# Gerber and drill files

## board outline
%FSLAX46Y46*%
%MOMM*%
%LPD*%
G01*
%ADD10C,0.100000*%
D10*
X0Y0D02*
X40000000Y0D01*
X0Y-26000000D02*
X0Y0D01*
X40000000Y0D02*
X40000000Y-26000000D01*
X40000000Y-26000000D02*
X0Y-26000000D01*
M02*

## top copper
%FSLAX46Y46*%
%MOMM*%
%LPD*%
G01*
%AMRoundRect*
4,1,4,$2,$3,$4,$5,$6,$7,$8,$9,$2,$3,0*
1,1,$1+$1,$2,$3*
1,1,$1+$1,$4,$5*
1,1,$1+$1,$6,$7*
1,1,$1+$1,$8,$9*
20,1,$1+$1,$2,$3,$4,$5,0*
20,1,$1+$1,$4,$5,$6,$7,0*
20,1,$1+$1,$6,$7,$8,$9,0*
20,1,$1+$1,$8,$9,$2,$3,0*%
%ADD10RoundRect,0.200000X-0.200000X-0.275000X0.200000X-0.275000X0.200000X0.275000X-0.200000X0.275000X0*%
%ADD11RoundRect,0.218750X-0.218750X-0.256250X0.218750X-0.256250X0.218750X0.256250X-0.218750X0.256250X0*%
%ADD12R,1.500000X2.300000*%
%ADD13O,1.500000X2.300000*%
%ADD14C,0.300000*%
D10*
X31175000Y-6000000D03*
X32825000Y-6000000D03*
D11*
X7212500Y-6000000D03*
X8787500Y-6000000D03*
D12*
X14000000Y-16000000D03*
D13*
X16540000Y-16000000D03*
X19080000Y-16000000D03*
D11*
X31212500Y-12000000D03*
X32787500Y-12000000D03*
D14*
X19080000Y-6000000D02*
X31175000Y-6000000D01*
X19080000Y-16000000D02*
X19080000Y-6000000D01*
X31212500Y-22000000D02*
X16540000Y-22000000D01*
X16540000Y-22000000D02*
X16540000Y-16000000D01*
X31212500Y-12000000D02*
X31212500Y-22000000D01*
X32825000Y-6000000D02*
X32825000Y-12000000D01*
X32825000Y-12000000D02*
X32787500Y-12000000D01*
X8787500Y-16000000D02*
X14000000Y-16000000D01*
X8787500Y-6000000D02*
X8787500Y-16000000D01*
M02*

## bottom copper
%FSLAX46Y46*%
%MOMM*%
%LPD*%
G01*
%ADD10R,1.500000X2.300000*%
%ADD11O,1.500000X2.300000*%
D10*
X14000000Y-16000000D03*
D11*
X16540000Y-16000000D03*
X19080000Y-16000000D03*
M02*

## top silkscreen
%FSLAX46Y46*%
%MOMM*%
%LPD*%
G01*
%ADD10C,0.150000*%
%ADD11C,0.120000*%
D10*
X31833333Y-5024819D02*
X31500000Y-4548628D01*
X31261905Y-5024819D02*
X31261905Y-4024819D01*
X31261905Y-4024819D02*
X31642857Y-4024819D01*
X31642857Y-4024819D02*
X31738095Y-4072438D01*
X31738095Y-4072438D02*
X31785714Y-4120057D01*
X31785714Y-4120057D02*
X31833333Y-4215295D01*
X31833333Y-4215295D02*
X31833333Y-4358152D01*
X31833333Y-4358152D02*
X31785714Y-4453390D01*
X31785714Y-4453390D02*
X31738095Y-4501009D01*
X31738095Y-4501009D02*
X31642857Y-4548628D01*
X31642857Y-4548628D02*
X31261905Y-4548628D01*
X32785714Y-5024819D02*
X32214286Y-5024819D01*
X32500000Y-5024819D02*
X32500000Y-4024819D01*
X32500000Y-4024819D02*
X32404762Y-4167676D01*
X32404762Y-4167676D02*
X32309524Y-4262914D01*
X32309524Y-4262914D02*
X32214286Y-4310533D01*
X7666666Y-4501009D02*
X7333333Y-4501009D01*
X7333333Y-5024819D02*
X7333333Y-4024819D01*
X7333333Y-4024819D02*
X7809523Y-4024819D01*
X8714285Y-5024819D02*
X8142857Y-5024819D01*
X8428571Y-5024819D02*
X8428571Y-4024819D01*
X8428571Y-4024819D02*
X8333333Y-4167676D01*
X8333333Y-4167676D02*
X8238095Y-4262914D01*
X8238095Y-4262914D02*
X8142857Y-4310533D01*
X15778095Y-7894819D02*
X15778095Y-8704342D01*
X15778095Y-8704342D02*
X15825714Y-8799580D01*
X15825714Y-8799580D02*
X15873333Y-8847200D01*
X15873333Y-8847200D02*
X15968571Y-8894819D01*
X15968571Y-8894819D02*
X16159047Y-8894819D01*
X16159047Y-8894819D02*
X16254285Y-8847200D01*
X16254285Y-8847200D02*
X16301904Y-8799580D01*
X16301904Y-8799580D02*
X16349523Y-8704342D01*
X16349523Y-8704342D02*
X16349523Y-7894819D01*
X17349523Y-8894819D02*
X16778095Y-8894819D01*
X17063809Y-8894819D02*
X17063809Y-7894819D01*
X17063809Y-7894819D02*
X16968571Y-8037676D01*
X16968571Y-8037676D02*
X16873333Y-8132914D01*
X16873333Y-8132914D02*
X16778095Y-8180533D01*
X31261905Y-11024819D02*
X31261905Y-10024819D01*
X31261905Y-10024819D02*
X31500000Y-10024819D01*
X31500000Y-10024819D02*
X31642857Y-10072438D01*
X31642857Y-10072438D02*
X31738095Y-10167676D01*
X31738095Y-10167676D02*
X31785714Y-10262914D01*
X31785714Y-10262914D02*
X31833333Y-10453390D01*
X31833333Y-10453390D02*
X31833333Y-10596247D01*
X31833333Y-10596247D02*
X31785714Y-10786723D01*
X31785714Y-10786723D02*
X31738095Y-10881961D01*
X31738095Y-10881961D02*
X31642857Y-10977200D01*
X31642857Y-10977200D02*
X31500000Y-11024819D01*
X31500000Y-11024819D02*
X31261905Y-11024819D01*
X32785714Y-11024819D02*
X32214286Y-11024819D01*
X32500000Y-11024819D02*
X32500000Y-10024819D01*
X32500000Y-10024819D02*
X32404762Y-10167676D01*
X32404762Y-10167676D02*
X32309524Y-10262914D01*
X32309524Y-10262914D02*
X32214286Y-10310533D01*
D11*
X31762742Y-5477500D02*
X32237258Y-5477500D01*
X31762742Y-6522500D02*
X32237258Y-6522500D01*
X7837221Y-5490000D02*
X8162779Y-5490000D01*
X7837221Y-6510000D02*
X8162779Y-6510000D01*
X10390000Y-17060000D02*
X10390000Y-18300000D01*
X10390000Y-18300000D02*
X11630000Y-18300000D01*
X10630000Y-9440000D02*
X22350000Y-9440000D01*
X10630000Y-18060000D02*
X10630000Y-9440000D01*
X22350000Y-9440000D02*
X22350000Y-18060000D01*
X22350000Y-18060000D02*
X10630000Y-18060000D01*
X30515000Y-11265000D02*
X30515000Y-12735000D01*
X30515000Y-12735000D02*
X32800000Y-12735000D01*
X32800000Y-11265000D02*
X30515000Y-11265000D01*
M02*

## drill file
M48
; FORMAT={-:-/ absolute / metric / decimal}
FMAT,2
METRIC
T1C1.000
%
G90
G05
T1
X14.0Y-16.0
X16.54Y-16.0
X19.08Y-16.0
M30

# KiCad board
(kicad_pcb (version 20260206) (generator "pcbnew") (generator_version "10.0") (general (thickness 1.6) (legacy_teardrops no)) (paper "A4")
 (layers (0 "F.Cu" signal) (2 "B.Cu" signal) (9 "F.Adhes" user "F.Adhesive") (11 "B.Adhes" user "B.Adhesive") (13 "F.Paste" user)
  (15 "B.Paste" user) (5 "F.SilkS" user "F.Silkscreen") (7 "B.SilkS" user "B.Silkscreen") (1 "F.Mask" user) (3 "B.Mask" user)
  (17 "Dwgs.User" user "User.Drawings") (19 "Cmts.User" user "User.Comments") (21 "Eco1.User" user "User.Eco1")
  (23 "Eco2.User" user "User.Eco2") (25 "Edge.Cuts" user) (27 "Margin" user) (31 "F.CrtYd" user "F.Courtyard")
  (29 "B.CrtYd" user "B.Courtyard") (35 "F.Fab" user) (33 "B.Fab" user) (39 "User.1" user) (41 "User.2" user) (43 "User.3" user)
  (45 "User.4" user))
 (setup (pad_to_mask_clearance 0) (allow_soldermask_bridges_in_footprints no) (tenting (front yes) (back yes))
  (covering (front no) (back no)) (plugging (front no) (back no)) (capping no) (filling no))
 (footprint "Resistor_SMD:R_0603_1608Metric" (layer "F.Cu") (at 32 6)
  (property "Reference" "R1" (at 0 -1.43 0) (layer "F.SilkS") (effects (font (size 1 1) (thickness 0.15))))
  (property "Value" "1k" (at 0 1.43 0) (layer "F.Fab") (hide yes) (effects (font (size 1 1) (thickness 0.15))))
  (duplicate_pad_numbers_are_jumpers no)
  (fp_line (start -0.237258 -0.5225) (end 0.237258 -0.5225) (stroke (width 0.12) (type solid)) (layer "F.SilkS"))
  (fp_line (start -0.237258 0.5225) (end 0.237258 0.5225) (stroke (width 0.12) (type solid)) (layer "F.SilkS"))
  (pad "1" smd roundrect (at -0.825 0) (size 0.8 0.95) (layers "F.Cu" "F.Mask" "F.Paste") (roundrect_rratio 0.25) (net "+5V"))
  (pad "2" smd roundrect (at 0.825 0) (size 0.8 0.95) (layers "F.Cu" "F.Mask" "F.Paste") (roundrect_rratio 0.25) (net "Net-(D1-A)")))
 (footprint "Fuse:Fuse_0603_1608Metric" (layer "F.Cu") (at 8 6)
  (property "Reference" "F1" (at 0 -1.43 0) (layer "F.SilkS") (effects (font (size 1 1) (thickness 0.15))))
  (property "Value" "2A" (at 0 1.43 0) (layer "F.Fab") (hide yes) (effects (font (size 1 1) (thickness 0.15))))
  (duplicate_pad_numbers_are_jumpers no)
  (fp_line (start -0.162779 -0.51) (end 0.162779 -0.51) (stroke (width 0.12) (type solid)) (layer "F.SilkS"))
  (fp_line (start -0.162779 0.51) (end 0.162779 0.51) (stroke (width 0.12) (type solid)) (layer "F.SilkS"))
  (pad "1" smd roundrect (at -0.7875 0) (size 0.875 0.95) (layers "F.Cu" "F.Mask" "F.Paste") (roundrect_rratio 0.25) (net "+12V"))
  (pad "2" smd roundrect (at 0.7875 0) (size 0.875 0.95) (layers "F.Cu" "F.Mask" "F.Paste") (roundrect_rratio 0.25) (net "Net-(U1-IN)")))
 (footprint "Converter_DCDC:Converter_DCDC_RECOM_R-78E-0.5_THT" (layer "F.Cu") (at 14 16)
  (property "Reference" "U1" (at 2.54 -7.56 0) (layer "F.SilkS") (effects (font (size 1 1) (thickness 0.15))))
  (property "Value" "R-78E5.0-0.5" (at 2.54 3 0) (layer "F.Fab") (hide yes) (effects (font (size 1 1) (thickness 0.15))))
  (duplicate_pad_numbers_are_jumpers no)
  (fp_line (start -3.61 1.06) (end -3.61 2.3) (stroke (width 0.12) (type solid)) (layer "F.SilkS"))
  (fp_line (start -3.61 2.3) (end -2.37 2.3) (stroke (width 0.12) (type solid)) (layer "F.SilkS"))
  (fp_line (start -3.37 -6.56) (end 8.35 -6.56) (stroke (width 0.12) (type solid)) (layer "F.SilkS"))
  (fp_line (start -3.37 2.06) (end -3.37 -6.56) (stroke (width 0.12) (type solid)) (layer "F.SilkS"))
  (fp_line (start 8.35 -6.56) (end 8.35 2.06) (stroke (width 0.12) (type solid)) (layer "F.SilkS"))
  (fp_line (start 8.35 2.06) (end -3.37 2.06) (stroke (width 0.12) (type solid)) (layer "F.SilkS"))
  (pad "1" thru_hole rect (at 0 0) (size 1.5 2.3) (drill 1) (layers "*.Cu" "*.Mask") (remove_unused_layers no) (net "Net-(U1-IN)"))
  (pad "2" thru_hole oval (at 2.54 0) (size 1.5 2.3) (drill 1) (layers "*.Cu" "*.Mask") (remove_unused_layers no) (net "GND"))
  (pad "3" thru_hole oval (at 5.08 0) (size 1.5 2.3) (drill 1) (layers "*.Cu" "*.Mask") (remove_unused_layers no) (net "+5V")))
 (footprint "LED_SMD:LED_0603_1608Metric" (layer "F.Cu") (at 32 12)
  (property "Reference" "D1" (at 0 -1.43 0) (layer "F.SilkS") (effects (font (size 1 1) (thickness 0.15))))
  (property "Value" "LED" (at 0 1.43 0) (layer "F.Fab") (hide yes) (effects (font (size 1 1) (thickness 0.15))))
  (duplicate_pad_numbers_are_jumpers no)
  (fp_line (start -1.485 -0.735) (end -1.485 0.735) (stroke (width 0.12) (type solid)) (layer "F.SilkS"))
  (fp_line (start -1.485 0.735) (end 0.8 0.735) (stroke (width 0.12) (type solid)) (layer "F.SilkS"))
  (fp_line (start 0.8 -0.735) (end -1.485 -0.735) (stroke (width 0.12) (type solid)) (layer "F.SilkS"))
  (pad "1" smd roundrect (at -0.7875 0) (size 0.875 0.95) (layers "F.Cu" "F.Mask" "F.Paste") (roundrect_rratio 0.25) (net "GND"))
  (pad "2" smd roundrect (at 0.7875 0) (size 0.875 0.95) (layers "F.Cu" "F.Mask" "F.Paste") (roundrect_rratio 0.25) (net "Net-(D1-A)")))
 (gr_line (start 0 0) (end 40 0) (stroke (width 0.1) (type default)) (layer "Edge.Cuts"))
 (gr_line (start 0 26) (end 0 0) (stroke (width 0.1) (type default)) (layer "Edge.Cuts"))
 (gr_line (start 40 0) (end 40 26) (stroke (width 0.1) (type default)) (layer "Edge.Cuts"))
 (gr_line (start 40 26) (end 0 26) (stroke (width 0.1) (type default)) (layer "Edge.Cuts"))
 (segment (start 19.08 6) (end 31.175 6) (width 0.3) (layer "F.Cu") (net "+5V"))
 (segment (start 19.08 16) (end 19.08 6) (width 0.3) (layer "F.Cu") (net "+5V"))
 (segment (start 31.2125 22) (end 16.54 22) (width 0.3) (layer "F.Cu") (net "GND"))
 (segment (start 16.54 22) (end 16.54 16) (width 0.3) (layer "F.Cu") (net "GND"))
 (segment (start 31.2125 12) (end 31.2125 22) (width 0.3) (layer "F.Cu") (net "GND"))
 (segment (start 32.825 6) (end 32.825 12) (width 0.3) (layer "F.Cu") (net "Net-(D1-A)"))
 (segment (start 32.825 12) (end 32.7875 12) (width 0.3) (layer "F.Cu") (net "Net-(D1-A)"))
 (segment (start 8.7875 16) (end 14 16) (width 0.3) (layer "F.Cu") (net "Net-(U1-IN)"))
 (segment (start 8.7875 6) (end 8.7875 16) (width 0.3) (layer "F.Cu") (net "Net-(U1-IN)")))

